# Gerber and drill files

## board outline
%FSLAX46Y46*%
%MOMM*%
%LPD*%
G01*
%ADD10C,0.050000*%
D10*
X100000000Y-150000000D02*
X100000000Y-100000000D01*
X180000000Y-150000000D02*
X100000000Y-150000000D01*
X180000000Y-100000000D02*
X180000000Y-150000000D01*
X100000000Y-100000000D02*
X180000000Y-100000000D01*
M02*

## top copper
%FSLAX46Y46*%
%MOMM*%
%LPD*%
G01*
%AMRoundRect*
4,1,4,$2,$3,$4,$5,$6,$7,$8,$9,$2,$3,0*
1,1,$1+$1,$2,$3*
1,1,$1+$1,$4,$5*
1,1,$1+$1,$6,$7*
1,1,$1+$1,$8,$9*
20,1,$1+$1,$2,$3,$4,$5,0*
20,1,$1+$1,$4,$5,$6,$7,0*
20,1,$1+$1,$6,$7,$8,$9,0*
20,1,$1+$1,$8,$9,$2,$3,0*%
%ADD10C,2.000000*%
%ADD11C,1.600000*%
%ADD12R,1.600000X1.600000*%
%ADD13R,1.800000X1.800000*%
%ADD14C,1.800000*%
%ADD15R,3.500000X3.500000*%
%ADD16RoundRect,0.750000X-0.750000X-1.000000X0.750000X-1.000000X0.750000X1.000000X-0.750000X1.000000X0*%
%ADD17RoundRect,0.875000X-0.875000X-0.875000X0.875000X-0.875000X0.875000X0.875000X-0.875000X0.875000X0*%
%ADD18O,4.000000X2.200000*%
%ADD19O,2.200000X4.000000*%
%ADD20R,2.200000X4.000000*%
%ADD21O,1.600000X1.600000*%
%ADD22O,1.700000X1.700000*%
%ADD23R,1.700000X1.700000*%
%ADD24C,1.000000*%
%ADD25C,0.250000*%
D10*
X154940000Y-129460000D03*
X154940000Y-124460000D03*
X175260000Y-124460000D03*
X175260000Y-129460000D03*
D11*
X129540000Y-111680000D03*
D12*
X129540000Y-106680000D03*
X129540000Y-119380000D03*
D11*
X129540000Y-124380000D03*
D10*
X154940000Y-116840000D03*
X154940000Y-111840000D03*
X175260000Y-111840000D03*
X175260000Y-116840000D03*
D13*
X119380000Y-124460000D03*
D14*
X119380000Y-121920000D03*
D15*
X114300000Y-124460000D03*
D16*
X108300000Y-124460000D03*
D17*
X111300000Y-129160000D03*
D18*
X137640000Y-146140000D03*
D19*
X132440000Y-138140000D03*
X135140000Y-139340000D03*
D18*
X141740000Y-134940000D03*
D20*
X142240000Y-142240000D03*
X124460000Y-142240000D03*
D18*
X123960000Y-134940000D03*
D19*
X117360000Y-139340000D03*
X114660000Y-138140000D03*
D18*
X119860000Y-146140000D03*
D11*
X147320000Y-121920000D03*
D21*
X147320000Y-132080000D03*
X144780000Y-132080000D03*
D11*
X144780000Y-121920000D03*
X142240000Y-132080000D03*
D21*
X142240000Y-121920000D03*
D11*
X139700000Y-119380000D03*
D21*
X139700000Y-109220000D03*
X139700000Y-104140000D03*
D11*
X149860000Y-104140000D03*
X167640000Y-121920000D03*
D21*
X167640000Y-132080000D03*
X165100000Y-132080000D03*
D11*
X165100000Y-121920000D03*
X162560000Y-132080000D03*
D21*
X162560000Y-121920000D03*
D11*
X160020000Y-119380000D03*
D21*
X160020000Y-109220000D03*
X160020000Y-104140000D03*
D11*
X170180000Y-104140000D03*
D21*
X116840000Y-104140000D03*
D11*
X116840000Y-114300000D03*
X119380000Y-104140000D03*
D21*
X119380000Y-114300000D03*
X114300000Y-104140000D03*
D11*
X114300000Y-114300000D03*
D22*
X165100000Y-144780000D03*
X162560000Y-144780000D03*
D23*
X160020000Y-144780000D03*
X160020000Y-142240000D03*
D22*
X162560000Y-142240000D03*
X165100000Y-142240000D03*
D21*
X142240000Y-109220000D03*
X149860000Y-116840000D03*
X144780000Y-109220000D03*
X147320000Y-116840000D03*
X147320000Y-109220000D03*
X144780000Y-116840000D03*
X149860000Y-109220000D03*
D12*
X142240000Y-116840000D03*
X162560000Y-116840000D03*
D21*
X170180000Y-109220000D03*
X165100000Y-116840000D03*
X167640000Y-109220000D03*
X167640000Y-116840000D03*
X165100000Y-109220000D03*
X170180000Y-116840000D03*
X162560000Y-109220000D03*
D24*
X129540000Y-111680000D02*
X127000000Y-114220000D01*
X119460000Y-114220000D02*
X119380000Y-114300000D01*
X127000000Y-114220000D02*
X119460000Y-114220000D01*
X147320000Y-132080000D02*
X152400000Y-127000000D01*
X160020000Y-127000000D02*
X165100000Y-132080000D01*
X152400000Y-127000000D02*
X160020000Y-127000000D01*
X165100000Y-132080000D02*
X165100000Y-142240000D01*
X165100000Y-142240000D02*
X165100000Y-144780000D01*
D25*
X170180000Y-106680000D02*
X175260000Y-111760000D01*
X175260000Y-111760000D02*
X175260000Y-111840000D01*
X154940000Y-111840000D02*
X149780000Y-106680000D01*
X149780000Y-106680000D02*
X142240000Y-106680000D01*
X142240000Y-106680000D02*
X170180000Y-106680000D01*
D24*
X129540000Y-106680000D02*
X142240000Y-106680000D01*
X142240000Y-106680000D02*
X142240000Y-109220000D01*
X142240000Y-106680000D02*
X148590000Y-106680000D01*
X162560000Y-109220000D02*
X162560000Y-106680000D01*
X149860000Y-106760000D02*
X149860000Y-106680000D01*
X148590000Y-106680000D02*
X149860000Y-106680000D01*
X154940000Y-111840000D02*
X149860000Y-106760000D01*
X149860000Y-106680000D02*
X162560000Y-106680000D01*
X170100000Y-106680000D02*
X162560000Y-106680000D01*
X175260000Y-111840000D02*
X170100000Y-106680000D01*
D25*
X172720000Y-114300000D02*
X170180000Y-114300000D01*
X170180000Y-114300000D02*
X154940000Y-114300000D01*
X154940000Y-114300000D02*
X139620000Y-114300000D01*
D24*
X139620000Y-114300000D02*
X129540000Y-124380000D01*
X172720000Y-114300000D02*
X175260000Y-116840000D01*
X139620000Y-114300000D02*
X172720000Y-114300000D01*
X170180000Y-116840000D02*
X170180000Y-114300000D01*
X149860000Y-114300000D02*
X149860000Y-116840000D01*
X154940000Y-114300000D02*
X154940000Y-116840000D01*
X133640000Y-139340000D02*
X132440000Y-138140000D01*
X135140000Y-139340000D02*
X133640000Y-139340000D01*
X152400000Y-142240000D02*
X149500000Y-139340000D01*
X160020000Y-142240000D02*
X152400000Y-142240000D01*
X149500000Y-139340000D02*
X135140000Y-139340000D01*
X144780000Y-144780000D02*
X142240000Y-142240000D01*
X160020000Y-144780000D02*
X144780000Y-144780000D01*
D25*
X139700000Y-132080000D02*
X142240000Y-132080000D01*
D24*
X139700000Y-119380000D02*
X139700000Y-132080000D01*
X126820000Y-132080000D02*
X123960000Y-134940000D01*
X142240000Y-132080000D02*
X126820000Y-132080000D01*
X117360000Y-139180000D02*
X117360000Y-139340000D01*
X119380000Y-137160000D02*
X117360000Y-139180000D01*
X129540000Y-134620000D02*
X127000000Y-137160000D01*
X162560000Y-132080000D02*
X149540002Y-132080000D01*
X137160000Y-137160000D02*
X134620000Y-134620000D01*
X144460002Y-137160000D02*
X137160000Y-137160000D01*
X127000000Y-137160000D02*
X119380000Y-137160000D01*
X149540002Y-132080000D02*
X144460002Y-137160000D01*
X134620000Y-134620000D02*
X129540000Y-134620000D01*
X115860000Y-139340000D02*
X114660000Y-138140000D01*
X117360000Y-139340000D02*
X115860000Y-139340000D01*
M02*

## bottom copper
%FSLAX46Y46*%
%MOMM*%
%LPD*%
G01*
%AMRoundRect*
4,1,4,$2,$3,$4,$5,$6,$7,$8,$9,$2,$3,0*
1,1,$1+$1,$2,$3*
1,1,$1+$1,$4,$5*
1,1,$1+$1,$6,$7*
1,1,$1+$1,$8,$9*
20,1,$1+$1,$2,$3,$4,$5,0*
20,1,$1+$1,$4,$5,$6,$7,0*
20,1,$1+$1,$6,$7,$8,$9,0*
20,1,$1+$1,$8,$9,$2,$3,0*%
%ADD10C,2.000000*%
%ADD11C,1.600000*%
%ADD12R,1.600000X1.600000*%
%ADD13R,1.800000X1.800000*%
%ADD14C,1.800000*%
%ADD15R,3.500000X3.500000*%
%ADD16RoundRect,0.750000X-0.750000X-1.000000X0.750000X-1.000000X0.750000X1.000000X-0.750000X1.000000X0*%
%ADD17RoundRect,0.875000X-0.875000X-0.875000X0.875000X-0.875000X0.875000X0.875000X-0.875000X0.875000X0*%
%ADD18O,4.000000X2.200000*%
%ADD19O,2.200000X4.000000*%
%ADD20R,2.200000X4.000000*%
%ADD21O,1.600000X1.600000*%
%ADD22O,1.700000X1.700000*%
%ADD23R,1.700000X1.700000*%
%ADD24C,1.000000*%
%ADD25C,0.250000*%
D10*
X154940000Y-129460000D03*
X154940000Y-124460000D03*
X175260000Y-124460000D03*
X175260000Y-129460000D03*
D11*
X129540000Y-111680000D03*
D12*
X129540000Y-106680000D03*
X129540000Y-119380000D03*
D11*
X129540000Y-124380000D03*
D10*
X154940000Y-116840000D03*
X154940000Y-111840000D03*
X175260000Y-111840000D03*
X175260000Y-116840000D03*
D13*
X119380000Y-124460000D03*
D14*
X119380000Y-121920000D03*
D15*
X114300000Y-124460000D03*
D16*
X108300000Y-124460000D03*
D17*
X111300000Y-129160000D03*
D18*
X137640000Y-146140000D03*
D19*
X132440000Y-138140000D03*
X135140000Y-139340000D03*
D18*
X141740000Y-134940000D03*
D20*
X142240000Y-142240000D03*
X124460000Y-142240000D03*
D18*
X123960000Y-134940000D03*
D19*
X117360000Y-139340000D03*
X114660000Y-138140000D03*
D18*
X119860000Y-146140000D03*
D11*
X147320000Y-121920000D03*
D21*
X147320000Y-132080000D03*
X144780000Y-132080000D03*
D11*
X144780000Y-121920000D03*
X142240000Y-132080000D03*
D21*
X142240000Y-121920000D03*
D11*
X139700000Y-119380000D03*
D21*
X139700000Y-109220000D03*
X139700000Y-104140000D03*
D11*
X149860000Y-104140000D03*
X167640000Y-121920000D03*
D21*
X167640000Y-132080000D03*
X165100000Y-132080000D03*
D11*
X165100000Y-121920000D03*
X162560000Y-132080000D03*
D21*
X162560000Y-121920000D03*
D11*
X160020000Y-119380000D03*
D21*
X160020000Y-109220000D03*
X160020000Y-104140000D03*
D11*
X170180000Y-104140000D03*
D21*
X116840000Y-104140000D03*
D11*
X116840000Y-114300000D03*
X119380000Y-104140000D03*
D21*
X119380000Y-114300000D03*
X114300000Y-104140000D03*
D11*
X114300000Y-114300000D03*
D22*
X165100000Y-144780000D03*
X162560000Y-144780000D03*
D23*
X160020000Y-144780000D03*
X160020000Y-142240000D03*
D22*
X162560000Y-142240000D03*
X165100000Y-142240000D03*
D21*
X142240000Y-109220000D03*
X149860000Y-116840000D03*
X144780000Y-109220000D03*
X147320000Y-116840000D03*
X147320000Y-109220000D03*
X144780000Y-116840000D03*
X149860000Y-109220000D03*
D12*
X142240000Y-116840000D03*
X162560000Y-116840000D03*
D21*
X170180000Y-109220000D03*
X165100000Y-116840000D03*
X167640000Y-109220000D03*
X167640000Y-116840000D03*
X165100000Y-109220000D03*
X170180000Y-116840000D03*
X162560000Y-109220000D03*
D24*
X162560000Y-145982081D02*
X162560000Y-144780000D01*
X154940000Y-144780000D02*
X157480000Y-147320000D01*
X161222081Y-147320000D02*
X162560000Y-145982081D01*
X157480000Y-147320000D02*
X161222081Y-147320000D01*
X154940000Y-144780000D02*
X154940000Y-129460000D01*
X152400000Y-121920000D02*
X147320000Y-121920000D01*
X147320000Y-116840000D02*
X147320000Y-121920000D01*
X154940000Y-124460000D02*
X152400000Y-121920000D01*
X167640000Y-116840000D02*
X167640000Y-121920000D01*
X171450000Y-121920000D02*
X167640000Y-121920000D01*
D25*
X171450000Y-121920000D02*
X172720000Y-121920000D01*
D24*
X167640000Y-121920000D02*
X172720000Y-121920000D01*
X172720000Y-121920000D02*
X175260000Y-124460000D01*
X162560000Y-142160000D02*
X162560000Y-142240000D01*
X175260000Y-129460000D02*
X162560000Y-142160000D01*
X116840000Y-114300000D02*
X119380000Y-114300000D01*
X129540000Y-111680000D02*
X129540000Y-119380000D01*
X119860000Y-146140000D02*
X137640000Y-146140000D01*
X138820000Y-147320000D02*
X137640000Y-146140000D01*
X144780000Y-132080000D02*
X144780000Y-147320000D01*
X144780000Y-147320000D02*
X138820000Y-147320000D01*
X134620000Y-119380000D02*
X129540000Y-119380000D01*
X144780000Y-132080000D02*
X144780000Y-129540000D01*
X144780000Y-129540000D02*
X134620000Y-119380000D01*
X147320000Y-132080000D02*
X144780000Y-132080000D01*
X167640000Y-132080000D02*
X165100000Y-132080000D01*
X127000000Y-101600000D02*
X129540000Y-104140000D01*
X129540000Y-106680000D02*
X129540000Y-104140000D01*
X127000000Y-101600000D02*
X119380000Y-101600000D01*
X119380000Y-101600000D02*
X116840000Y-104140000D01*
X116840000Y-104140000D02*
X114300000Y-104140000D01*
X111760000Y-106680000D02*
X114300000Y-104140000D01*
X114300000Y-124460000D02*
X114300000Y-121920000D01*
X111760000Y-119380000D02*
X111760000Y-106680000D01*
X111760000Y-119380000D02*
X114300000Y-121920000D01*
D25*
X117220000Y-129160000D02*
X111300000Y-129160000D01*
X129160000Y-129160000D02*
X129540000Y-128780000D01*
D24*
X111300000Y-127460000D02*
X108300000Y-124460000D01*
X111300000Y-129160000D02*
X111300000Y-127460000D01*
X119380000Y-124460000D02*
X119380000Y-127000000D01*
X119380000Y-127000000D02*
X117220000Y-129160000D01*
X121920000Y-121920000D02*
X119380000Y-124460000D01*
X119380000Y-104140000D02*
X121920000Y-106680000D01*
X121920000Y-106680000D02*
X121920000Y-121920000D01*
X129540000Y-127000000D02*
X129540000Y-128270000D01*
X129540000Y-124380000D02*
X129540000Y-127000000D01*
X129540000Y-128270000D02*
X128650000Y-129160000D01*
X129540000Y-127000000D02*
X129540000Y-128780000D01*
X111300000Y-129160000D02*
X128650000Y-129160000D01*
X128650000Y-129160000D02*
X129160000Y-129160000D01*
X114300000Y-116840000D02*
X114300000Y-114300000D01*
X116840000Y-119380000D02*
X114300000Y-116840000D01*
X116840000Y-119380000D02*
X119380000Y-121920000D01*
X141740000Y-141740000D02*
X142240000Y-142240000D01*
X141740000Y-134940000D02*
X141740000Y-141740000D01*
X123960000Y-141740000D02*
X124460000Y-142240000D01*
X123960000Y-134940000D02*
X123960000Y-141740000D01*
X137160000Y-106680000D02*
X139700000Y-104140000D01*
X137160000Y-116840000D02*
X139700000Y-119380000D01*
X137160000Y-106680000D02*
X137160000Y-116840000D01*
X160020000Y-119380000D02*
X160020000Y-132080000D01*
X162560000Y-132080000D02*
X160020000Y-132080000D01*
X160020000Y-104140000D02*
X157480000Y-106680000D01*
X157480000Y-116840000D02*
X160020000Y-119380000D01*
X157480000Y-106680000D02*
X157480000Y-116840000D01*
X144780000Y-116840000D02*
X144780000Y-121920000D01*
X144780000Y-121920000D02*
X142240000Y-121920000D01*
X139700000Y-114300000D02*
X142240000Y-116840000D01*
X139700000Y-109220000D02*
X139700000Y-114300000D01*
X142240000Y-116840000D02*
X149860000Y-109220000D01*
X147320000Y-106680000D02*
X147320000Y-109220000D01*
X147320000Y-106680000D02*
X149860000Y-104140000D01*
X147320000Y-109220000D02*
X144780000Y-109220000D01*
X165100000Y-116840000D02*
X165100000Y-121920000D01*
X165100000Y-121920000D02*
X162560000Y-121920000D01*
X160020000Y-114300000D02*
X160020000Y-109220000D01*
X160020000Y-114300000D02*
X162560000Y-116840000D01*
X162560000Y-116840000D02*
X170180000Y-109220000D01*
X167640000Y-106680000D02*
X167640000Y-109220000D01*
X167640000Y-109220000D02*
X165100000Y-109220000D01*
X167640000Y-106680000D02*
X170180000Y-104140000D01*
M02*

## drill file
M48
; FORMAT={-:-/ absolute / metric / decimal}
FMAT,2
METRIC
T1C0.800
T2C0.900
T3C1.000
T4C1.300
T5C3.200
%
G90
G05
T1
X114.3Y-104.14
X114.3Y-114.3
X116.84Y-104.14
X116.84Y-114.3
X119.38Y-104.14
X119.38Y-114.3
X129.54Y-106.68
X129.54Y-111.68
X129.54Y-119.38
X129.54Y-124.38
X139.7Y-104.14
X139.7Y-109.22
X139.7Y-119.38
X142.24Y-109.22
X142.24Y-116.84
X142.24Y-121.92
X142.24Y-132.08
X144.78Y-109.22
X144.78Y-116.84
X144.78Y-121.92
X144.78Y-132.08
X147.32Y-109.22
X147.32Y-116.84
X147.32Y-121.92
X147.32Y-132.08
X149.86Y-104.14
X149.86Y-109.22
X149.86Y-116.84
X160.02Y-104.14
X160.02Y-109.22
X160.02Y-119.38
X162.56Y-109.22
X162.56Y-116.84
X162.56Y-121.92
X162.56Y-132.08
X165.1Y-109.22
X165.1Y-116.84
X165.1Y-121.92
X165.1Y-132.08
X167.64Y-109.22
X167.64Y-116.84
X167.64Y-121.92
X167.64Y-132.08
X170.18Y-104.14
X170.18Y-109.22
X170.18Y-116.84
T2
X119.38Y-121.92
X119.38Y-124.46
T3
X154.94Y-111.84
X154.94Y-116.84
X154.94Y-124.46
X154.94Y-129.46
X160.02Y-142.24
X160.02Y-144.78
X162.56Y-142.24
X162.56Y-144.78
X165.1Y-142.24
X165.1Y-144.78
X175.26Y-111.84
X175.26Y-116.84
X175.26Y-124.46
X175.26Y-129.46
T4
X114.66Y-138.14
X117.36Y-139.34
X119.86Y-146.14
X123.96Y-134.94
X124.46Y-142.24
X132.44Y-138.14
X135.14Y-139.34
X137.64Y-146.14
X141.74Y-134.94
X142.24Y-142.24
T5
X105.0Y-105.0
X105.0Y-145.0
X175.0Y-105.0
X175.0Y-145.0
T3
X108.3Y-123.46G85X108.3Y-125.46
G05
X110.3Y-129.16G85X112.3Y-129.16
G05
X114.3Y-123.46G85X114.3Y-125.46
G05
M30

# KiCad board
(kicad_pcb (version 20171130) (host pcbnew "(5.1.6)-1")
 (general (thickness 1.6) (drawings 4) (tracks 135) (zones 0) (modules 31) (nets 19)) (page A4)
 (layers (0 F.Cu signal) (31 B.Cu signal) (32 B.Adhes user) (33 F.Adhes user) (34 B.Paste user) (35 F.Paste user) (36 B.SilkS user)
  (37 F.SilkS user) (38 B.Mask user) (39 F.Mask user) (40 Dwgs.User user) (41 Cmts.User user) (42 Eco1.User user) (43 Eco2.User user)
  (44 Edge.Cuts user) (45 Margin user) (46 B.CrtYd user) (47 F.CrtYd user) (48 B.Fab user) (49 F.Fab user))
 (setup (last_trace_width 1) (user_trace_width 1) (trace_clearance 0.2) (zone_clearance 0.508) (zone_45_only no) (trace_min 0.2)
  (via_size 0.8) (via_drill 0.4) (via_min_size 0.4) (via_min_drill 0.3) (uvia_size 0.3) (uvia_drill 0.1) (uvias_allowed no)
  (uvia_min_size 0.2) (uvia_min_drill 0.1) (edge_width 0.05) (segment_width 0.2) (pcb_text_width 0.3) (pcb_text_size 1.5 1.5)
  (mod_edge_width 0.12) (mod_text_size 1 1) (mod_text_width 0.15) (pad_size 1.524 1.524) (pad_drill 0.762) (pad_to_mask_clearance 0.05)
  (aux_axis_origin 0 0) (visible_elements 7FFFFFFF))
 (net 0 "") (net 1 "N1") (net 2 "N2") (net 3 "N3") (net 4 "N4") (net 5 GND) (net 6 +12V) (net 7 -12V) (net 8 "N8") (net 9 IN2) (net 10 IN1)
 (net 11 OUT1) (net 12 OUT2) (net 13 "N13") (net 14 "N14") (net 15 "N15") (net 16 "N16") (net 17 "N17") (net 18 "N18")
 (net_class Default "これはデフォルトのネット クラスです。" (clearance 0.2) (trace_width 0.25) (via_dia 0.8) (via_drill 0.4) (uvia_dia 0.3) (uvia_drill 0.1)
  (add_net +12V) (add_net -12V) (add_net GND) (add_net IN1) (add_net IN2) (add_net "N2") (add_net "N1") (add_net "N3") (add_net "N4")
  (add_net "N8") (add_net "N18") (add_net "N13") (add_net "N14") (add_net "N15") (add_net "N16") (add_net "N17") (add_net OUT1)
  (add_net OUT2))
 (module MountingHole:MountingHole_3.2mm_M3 (layer F.Cu) (at 175 105)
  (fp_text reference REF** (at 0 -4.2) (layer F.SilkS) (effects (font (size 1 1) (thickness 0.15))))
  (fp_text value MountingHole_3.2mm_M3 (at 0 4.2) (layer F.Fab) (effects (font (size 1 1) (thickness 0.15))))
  (pad 1 np_thru_hole circle (at 0 0) (size 3.2 3.2) (drill 3.2) (layers *.Cu *.Mask)))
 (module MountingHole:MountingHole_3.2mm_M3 (layer F.Cu) (at 175 145)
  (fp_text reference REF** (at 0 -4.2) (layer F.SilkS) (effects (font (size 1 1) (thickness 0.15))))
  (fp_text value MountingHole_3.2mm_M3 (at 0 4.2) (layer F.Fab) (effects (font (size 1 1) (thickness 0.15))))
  (pad 1 np_thru_hole circle (at 0 0) (size 3.2 3.2) (drill 3.2) (layers *.Cu *.Mask)))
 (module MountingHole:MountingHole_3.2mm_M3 (layer F.Cu) (at 105 145)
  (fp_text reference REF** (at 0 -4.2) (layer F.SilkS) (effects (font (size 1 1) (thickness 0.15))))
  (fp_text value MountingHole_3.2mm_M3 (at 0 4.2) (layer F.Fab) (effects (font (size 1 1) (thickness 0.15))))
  (pad 1 np_thru_hole circle (at 0 0) (size 3.2 3.2) (drill 3.2) (layers *.Cu *.Mask)))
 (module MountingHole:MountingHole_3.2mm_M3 (layer F.Cu) (at 105 105)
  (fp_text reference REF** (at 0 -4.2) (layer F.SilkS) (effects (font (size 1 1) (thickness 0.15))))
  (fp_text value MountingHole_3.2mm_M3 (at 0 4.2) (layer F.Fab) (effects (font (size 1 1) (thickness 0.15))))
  (pad 1 np_thru_hole circle (at 0 0) (size 3.2 3.2) (drill 3.2) (layers *.Cu *.Mask)))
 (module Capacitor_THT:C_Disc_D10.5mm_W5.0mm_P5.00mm (layer F.Cu) (at 154.94 124.46 270)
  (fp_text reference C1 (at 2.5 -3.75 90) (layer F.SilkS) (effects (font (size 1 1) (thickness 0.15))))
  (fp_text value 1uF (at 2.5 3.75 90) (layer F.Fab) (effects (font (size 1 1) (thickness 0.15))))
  (pad 2 thru_hole circle (at 5 0 270) (size 2 2) (drill 1) (layers *.Cu *.Mask) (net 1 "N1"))
  (pad 1 thru_hole circle (at 0 0 270) (size 2 2) (drill 1) (layers *.Cu *.Mask) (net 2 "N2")))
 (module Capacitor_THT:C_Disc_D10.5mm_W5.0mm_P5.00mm (layer F.Cu) (at 175.26 124.46 270)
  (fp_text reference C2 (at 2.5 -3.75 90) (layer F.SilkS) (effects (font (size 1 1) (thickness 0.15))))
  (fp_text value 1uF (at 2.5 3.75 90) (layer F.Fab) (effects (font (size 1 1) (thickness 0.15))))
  (pad 1 thru_hole circle (at 0 0 270) (size 2 2) (drill 1) (layers *.Cu *.Mask) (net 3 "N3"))
  (pad 2 thru_hole circle (at 5 0 270) (size 2 2) (drill 1) (layers *.Cu *.Mask) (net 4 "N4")))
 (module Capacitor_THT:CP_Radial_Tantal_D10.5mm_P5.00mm (layer F.Cu) (at 129.54 106.68 270)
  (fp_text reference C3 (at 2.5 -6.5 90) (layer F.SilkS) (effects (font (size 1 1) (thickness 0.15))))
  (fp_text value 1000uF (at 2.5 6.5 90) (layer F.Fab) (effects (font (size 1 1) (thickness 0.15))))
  (pad 2 thru_hole circle (at 5 0 270) (size 1.6 1.6) (drill 0.8) (layers *.Cu *.Mask) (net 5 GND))
  (pad 1 thru_hole rect (at 0 0 270) (size 1.6 1.6) (drill 0.8) (layers *.Cu *.Mask) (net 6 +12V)))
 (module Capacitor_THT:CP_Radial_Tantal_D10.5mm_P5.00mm (layer F.Cu) (at 129.54 119.38 270)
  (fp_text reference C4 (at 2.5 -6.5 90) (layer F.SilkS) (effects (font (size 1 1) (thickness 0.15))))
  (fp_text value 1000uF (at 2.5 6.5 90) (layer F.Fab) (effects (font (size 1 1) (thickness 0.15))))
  (pad 1 thru_hole rect (at 0 0 270) (size 1.6 1.6) (drill 0.8) (layers *.Cu *.Mask) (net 5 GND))
  (pad 2 thru_hole circle (at 5 0 270) (size 1.6 1.6) (drill 0.8) (layers *.Cu *.Mask) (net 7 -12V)))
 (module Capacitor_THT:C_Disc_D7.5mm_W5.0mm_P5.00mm (layer F.Cu) (at 154.94 116.84 90)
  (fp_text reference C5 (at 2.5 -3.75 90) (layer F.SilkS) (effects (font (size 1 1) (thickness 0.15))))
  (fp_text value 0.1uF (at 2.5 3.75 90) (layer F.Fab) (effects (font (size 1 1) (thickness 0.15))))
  (pad 1 thru_hole circle (at 0 0 90) (size 2 2) (drill 1) (layers *.Cu *.Mask) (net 7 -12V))
  (pad 2 thru_hole circle (at 5 0 90) (size 2 2) (drill 1) (layers *.Cu *.Mask) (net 6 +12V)))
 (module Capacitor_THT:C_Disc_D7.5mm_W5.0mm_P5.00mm (layer F.Cu) (at 175.26 116.84 90)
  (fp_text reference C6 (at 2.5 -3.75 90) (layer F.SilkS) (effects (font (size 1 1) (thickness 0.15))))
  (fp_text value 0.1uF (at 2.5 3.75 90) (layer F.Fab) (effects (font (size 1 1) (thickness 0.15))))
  (pad 2 thru_hole circle (at 5 0 90) (size 2 2) (drill 1) (layers *.Cu *.Mask) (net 6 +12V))
  (pad 1 thru_hole circle (at 0 0 90) (size 2 2) (drill 1) (layers *.Cu *.Mask) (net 7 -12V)))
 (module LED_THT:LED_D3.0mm (layer F.Cu) (at 119.38 124.46 90)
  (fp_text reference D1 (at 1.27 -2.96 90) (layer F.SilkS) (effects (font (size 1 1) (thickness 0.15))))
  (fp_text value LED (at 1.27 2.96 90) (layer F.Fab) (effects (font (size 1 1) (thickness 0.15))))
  (pad 1 thru_hole rect (at 0 0 90) (size 1.8 1.8) (drill 0.9) (layers *.Cu *.Mask) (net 7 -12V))
  (pad 2 thru_hole circle (at 2.54 0 90) (size 1.8 1.8) (drill 0.9) (layers *.Cu *.Mask) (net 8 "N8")))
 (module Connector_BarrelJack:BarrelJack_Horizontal (layer F.Cu) (at 114.3 124.46)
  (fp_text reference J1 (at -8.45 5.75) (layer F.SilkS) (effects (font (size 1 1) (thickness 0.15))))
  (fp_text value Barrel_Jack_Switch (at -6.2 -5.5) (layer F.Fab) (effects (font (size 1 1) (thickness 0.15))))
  (pad 1 thru_hole rect (at 0 0) (size 3.5 3.5) (drill oval 1 3) (layers *.Cu *.Mask) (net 6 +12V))
  (pad 2 thru_hole roundrect (at -6 0) (size 3 3.5) (drill oval 1 3) (layers *.Cu *.Mask) (roundrect_rratio 0.25) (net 7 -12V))
  (pad 3 thru_hole roundrect (at -3 4.7) (size 3.5 3.5) (drill oval 3 1) (layers *.Cu *.Mask) (roundrect_rratio 0.25) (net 7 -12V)))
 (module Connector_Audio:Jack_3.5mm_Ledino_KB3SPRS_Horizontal (layer F.Cu) (at 142.24 142.24 90)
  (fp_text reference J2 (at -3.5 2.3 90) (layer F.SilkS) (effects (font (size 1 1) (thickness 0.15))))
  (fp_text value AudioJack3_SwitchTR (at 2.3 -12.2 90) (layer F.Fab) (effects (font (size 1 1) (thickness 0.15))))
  (pad S thru_hole oval (at -3.9 -4.6 90) (size 2.2 4) (drill 1.3) (layers *.Cu *.Mask) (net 5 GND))
  (pad R thru_hole oval (at 4.1 -9.8 90) (size 4 2.2) (drill 1.3) (layers *.Cu *.Mask) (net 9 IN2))
  (pad RN thru_hole oval (at 2.9 -7.1 90) (size 4 2.2) (drill 1.3) (layers *.Cu *.Mask) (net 9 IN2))
  (pad TN thru_hole oval (at 7.3 -0.5 180) (size 4 2.2) (drill 1.3) (layers *.Cu *.Mask) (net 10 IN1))
  (pad T thru_hole rect (at 0 0 90) (size 4 2.2) (drill 1.3) (layers *.Cu *.Mask) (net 10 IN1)))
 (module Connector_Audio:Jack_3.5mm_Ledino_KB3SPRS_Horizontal (layer F.Cu) (at 124.46 142.24 90)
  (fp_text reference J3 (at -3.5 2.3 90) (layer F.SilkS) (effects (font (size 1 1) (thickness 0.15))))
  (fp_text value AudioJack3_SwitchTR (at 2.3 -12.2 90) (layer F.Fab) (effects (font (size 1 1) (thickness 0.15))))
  (pad T thru_hole rect (at 0 0 90) (size 4 2.2) (drill 1.3) (layers *.Cu *.Mask) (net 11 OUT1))
  (pad TN thru_hole oval (at 7.3 -0.5 180) (size 4 2.2) (drill 1.3) (layers *.Cu *.Mask) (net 11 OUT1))
  (pad RN thru_hole oval (at 2.9 -7.1 90) (size 4 2.2) (drill 1.3) (layers *.Cu *.Mask) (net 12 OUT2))
  (pad R thru_hole oval (at 4.1 -9.8 90) (size 4 2.2) (drill 1.3) (layers *.Cu *.Mask) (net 12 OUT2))
  (pad S thru_hole oval (at -3.9 -4.6 90) (size 2.2 4) (drill 1.3) (layers *.Cu *.Mask) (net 5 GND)))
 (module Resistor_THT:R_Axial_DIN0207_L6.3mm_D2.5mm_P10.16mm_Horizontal (layer F.Cu) (at 147.32 121.92 270)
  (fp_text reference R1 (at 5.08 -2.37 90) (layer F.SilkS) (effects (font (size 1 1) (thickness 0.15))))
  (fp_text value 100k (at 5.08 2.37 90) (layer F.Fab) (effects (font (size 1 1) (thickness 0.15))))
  (pad 1 thru_hole circle (at 0 0 270) (size 1.6 1.6) (drill 0.8) (layers *.Cu *.Mask) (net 2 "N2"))
  (pad 2 thru_hole oval (at 10.16 0 270) (size 1.6 1.6) (drill 0.8) (layers *.Cu *.Mask) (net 5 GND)))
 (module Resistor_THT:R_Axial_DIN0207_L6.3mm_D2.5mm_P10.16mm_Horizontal (layer F.Cu) (at 144.78 121.92 270)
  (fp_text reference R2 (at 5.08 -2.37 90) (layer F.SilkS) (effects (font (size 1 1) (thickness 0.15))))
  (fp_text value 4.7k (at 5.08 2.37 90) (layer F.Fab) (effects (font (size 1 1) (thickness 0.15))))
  (pad 2 thru_hole oval (at 10.16 0 270) (size 1.6 1.6) (drill 0.8) (layers *.Cu *.Mask) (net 5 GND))
  (pad 1 thru_hole circle (at 0 0 270) (size 1.6 1.6) (drill 0.8) (layers *.Cu *.Mask) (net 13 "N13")))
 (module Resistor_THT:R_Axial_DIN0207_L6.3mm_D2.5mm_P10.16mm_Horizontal (layer F.Cu) (at 142.24 132.08 90)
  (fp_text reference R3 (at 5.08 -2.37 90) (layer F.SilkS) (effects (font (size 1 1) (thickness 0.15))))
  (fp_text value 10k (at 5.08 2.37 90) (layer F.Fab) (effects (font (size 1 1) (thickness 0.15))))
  (pad 1 thru_hole circle (at 0 0 90) (size 1.6 1.6) (drill 0.8) (layers *.Cu *.Mask) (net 11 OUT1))
  (pad 2 thru_hole oval (at 10.16 0 90) (size 1.6 1.6) (drill 0.8) (layers *.Cu *.Mask) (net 13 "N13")))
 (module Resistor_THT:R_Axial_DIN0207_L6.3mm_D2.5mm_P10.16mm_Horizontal (layer F.Cu) (at 139.7 119.38 90)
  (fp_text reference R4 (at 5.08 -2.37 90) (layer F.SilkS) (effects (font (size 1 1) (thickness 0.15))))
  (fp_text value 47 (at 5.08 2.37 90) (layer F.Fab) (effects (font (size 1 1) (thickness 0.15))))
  (pad 1 thru_hole circle (at 0 0 90) (size 1.6 1.6) (drill 0.8) (layers *.Cu *.Mask) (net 11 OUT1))
  (pad 2 thru_hole oval (at 10.16 0 90) (size 1.6 1.6) (drill 0.8) (layers *.Cu *.Mask) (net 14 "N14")))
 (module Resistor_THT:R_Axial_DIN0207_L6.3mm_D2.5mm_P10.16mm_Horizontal (layer F.Cu) (at 149.86 104.14 180)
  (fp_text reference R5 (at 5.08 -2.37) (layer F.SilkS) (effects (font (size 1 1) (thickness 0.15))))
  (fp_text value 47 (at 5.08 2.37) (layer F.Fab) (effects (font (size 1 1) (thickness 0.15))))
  (pad 2 thru_hole oval (at 10.16 0 180) (size 1.6 1.6) (drill 0.8) (layers *.Cu *.Mask) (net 11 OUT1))
  (pad 1 thru_hole circle (at 0 0 180) (size 1.6 1.6) (drill 0.8) (layers *.Cu *.Mask) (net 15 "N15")))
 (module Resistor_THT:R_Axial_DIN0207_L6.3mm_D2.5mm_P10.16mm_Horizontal (layer F.Cu) (at 167.64 121.92 270)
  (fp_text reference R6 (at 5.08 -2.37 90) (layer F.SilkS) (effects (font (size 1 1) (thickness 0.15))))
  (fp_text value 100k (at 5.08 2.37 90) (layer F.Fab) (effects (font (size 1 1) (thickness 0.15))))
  (pad 1 thru_hole circle (at 0 0 270) (size 1.6 1.6) (drill 0.8) (layers *.Cu *.Mask) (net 3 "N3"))
  (pad 2 thru_hole oval (at 10.16 0 270) (size 1.6 1.6) (drill 0.8) (layers *.Cu *.Mask) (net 5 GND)))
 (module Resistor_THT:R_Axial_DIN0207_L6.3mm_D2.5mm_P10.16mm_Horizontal (layer F.Cu) (at 165.1 121.92 270)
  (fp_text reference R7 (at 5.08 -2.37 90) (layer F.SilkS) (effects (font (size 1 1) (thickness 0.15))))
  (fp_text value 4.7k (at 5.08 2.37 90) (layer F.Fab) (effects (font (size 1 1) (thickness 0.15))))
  (pad 2 thru_hole oval (at 10.16 0 270) (size 1.6 1.6) (drill 0.8) (layers *.Cu *.Mask) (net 5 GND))
  (pad 1 thru_hole circle (at 0 0 270) (size 1.6 1.6) (drill 0.8) (layers *.Cu *.Mask) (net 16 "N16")))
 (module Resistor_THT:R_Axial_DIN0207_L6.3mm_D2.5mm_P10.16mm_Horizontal (layer F.Cu) (at 162.56 132.08 90)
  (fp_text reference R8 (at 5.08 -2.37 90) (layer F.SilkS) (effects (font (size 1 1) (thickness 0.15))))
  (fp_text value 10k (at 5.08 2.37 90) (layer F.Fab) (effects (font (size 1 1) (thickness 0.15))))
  (pad 1 thru_hole circle (at 0 0 90) (size 1.6 1.6) (drill 0.8) (layers *.Cu *.Mask) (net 12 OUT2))
  (pad 2 thru_hole oval (at 10.16 0 90) (size 1.6 1.6) (drill 0.8) (layers *.Cu *.Mask) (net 16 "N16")))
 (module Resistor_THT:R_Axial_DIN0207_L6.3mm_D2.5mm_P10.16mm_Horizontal (layer F.Cu) (at 160.02 119.38 90)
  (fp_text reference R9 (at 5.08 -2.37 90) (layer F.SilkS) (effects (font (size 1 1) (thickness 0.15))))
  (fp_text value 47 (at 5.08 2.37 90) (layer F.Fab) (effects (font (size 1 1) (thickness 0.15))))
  (pad 1 thru_hole circle (at 0 0 90) (size 1.6 1.6) (drill 0.8) (layers *.Cu *.Mask) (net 12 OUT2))
  (pad 2 thru_hole oval (at 10.16 0 90) (size 1.6 1.6) (drill 0.8) (layers *.Cu *.Mask) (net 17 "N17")))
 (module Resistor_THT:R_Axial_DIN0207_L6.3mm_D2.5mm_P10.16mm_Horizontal (layer F.Cu) (at 170.18 104.14 180)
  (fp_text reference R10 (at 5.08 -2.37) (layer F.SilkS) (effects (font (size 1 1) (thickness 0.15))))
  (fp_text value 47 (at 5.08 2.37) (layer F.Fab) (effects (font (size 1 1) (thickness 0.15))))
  (pad 2 thru_hole oval (at 10.16 0 180) (size 1.6 1.6) (drill 0.8) (layers *.Cu *.Mask) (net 12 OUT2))
  (pad 1 thru_hole circle (at 0 0 180) (size 1.6 1.6) (drill 0.8) (layers *.Cu *.Mask) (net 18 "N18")))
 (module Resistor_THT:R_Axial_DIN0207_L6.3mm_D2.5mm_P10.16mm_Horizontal (layer F.Cu) (at 116.84 114.3 90)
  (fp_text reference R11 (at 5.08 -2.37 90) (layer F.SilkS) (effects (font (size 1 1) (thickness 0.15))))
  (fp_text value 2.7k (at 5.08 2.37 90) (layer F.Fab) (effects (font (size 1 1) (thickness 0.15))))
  (pad 2 thru_hole oval (at 10.16 0 90) (size 1.6 1.6) (drill 0.8) (layers *.Cu *.Mask) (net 6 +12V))
  (pad 1 thru_hole circle (at 0 0 90) (size 1.6 1.6) (drill 0.8) (layers *.Cu *.Mask) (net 5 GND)))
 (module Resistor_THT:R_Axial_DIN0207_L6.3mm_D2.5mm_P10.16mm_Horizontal (layer F.Cu) (at 119.38 104.14 270)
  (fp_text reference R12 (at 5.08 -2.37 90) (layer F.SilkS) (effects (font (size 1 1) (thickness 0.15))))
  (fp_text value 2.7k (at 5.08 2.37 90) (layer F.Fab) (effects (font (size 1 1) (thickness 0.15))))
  (pad 1 thru_hole circle (at 0 0 270) (size 1.6 1.6) (drill 0.8) (layers *.Cu *.Mask) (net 7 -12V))
  (pad 2 thru_hole oval (at 10.16 0 270) (size 1.6 1.6) (drill 0.8) (layers *.Cu *.Mask) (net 5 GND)))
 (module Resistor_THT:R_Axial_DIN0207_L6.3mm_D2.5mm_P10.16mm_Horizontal (layer F.Cu) (at 114.3 114.3 90)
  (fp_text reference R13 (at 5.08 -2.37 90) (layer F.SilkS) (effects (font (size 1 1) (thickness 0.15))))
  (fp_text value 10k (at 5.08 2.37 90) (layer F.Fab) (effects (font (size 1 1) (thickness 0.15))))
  (pad 2 thru_hole oval (at 10.16 0 90) (size 1.6 1.6) (drill 0.8) (layers *.Cu *.Mask) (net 6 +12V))
  (pad 1 thru_hole circle (at 0 0 90) (size 1.6 1.6) (drill 0.8) (layers *.Cu *.Mask) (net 8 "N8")))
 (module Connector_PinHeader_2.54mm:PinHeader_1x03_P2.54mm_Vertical (layer F.Cu) (at 160.02 144.78 90)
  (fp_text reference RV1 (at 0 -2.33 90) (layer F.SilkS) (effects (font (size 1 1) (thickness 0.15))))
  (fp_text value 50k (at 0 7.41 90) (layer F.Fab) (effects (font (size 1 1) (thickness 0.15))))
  (pad 3 thru_hole oval (at 0 5.08 90) (size 1.7 1.7) (drill 1) (layers *.Cu *.Mask) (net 5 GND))
  (pad 2 thru_hole oval (at 0 2.54 90) (size 1.7 1.7) (drill 1) (layers *.Cu *.Mask) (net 1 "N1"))
  (pad 1 thru_hole rect (at 0 0 90) (size 1.7 1.7) (drill 1) (layers *.Cu *.Mask) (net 10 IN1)))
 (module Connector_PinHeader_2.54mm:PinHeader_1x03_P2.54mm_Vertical (layer F.Cu) (at 160.02 142.24 90)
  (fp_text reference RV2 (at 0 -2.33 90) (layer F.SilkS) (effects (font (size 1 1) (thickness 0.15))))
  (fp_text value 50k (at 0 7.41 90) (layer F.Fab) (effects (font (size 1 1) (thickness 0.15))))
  (pad 1 thru_hole rect (at 0 0 90) (size 1.7 1.7) (drill 1) (layers *.Cu *.Mask) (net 9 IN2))
  (pad 2 thru_hole oval (at 0 2.54 90) (size 1.7 1.7) (drill 1) (layers *.Cu *.Mask) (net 4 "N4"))
  (pad 3 thru_hole oval (at 0 5.08 90) (size 1.7 1.7) (drill 1) (layers *.Cu *.Mask) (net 5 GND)))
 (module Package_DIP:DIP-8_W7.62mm (layer F.Cu) (at 142.24 116.84 90)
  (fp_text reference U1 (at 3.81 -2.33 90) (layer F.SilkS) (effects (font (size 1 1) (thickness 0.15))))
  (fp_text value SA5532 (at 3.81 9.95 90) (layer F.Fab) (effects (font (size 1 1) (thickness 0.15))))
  (pad 8 thru_hole oval (at 7.62 0 90) (size 1.6 1.6) (drill 0.8) (layers *.Cu *.Mask) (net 6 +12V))
  (pad 4 thru_hole oval (at 0 7.62 90) (size 1.6 1.6) (drill 0.8) (layers *.Cu *.Mask) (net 7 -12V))
  (pad 7 thru_hole oval (at 7.62 2.54 90) (size 1.6 1.6) (drill 0.8) (layers *.Cu *.Mask) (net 15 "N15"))
  (pad 3 thru_hole oval (at 0 5.08 90) (size 1.6 1.6) (drill 0.8) (layers *.Cu *.Mask) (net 2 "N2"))
  (pad 6 thru_hole oval (at 7.62 5.08 90) (size 1.6 1.6) (drill 0.8) (layers *.Cu *.Mask) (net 15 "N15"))
  (pad 2 thru_hole oval (at 0 2.54 90) (size 1.6 1.6) (drill 0.8) (layers *.Cu *.Mask) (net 13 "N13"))
  (pad 5 thru_hole oval (at 7.62 7.62 90) (size 1.6 1.6) (drill 0.8) (layers *.Cu *.Mask) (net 14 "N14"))
  (pad 1 thru_hole rect (at 0 0 90) (size 1.6 1.6) (drill 0.8) (layers *.Cu *.Mask) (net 14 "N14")))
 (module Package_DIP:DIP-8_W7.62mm (layer F.Cu) (at 162.56 116.84 90)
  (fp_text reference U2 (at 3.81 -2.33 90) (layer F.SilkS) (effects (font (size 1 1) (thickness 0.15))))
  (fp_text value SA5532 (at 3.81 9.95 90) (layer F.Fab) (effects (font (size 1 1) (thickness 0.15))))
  (pad 1 thru_hole rect (at 0 0 90) (size 1.6 1.6) (drill 0.8) (layers *.Cu *.Mask) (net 17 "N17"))
  (pad 5 thru_hole oval (at 7.62 7.62 90) (size 1.6 1.6) (drill 0.8) (layers *.Cu *.Mask) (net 17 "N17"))
  (pad 2 thru_hole oval (at 0 2.54 90) (size 1.6 1.6) (drill 0.8) (layers *.Cu *.Mask) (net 16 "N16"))
  (pad 6 thru_hole oval (at 7.62 5.08 90) (size 1.6 1.6) (drill 0.8) (layers *.Cu *.Mask) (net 18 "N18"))
  (pad 3 thru_hole oval (at 0 5.08 90) (size 1.6 1.6) (drill 0.8) (layers *.Cu *.Mask) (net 3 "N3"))
  (pad 7 thru_hole oval (at 7.62 2.54 90) (size 1.6 1.6) (drill 0.8) (layers *.Cu *.Mask) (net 18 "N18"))
  (pad 4 thru_hole oval (at 0 7.62 90) (size 1.6 1.6) (drill 0.8) (layers *.Cu *.Mask) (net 7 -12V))
  (pad 8 thru_hole oval (at 7.62 0 90) (size 1.6 1.6) (drill 0.8) (layers *.Cu *.Mask) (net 6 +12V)))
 (gr_line (start 100 150) (end 100 100) (layer Edge.Cuts) (width 0.05))
 (gr_line (start 180 150) (end 100 150) (layer Edge.Cuts) (width 0.05))
 (gr_line (start 180 100) (end 180 150) (layer Edge.Cuts) (width 0.05))
 (gr_line (start 100 100) (end 180 100) (layer Edge.Cuts) (width 0.05))
 (segment (start 162.56 145.982081) (end 162.56 144.78) (width 1) (layer B.Cu) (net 1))
 (segment (start 154.94 144.78) (end 157.48 147.32) (width 1) (layer B.Cu) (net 1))
 (segment (start 161.222081 147.32) (end 162.56 145.982081) (width 1) (layer B.Cu) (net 1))
 (segment (start 157.48 147.32) (end 161.222081 147.32) (width 1) (layer B.Cu) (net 1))
 (segment (start 154.94 144.78) (end 154.94 129.46) (width 1) (layer B.Cu) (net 1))
 (segment (start 152.4 121.92) (end 147.32 121.92) (width 1) (layer B.Cu) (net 2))
 (segment (start 147.32 116.84) (end 147.32 121.92) (width 1) (layer B.Cu) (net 2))
 (segment (start 154.94 124.46) (end 152.4 121.92) (width 1) (layer B.Cu) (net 2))
 (segment (start 167.64 116.84) (end 167.64 121.92) (width 1) (layer B.Cu) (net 3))
 (segment (start 171.45 121.92) (end 167.64 121.92) (width 1) (layer B.Cu) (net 3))
 (segment (start 171.45 121.92) (end 172.72 121.92) (width 0.25) (layer B.Cu) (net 3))
 (segment (start 167.64 121.92) (end 172.72 121.92) (width 1) (layer B.Cu) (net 3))
 (segment (start 172.72 121.92) (end 175.26 124.46) (width 1) (layer B.Cu) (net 3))
 (segment (start 162.56 142.16) (end 162.56 142.24) (width 1) (layer B.Cu) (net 4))
 (segment (start 175.26 129.46) (end 162.56 142.16) (width 1) (layer B.Cu) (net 4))
 (segment (start 116.84 114.3) (end 119.38 114.3) (width 1) (layer B.Cu) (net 5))
 (segment (start 129.54 111.68) (end 127 114.22) (width 1) (layer F.Cu) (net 5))
 (segment (start 119.46 114.22) (end 119.38 114.3) (width 1) (layer F.Cu) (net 5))
 (segment (start 127 114.22) (end 119.46 114.22) (width 1) (layer F.Cu) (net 5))
 (segment (start 129.54 111.68) (end 129.54 119.38) (width 1) (layer B.Cu) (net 5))
 (segment (start 119.86 146.14) (end 137.64 146.14) (width 1) (layer B.Cu) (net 5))
 (segment (start 138.82 147.32) (end 137.64 146.14) (width 1) (layer B.Cu) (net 5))
 (segment (start 144.78 132.08) (end 144.78 147.32) (width 1) (layer B.Cu) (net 5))
 (segment (start 144.78 147.32) (end 138.82 147.32) (width 1) (layer B.Cu) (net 5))
 (segment (start 134.62 119.38) (end 129.54 119.38) (width 1) (layer B.Cu) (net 5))
 (segment (start 144.78 132.08) (end 144.78 129.54) (width 1) (layer B.Cu) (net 5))
 (segment (start 144.78 129.54) (end 134.62 119.38) (width 1) (layer B.Cu) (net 5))
 (segment (start 147.32 132.08) (end 144.78 132.08) (width 1) (layer B.Cu) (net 5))
 (segment (start 167.64 132.08) (end 165.1 132.08) (width 1) (layer B.Cu) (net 5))
 (segment (start 147.32 132.08) (end 152.4 127) (width 1) (layer F.Cu) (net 5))
 (segment (start 160.02 127) (end 165.1 132.08) (width 1) (layer F.Cu) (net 5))
 (segment (start 152.4 127) (end 160.02 127) (width 1) (layer F.Cu) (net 5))
 (segment (start 165.1 132.08) (end 165.1 142.24) (width 1) (layer F.Cu) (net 5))
 (segment (start 165.1 142.24) (end 165.1 144.78) (width 1) (layer F.Cu) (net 5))
 (segment (start 170.18 106.68) (end 175.26 111.76) (width 0.25) (layer F.Cu) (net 6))
 (segment (start 175.26 111.76) (end 175.26 111.84) (width 0.25) (layer F.Cu) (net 6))
 (segment (start 154.94 111.84) (end 149.78 106.68) (width 0.25) (layer F.Cu) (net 6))
 (segment (start 149.78 106.68) (end 142.24 106.68) (width 0.25) (layer F.Cu) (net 6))
 (segment (start 142.24 106.68) (end 170.18 106.68) (width 0.25) (layer F.Cu) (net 6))
 (segment (start 127 101.6) (end 129.54 104.14) (width 1) (layer B.Cu) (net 6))
 (segment (start 129.54 106.68) (end 129.54 104.14) (width 1) (layer B.Cu) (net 6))
 (segment (start 127 101.6) (end 119.38 101.6) (width 1) (layer B.Cu) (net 6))
 (segment (start 119.38 101.6) (end 116.84 104.14) (width 1) (layer B.Cu) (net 6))
 (segment (start 116.84 104.14) (end 114.3 104.14) (width 1) (layer B.Cu) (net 6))
 (segment (start 111.76 106.68) (end 114.3 104.14) (width 1) (layer B.Cu) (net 6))
 (segment (start 114.3 124.46) (end 114.3 121.92) (width 1) (layer B.Cu) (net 6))
 (segment (start 111.76 119.38) (end 111.76 106.68) (width 1) (layer B.Cu) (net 6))
 (segment (start 111.76 119.38) (end 114.3 121.92) (width 1) (layer B.Cu) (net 6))
 (segment (start 129.54 106.68) (end 142.24 106.68) (width 1) (layer F.Cu) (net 6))
 (segment (start 142.24 106.68) (end 142.24 109.22) (width 1) (layer F.Cu) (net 6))
 (segment (start 142.24 106.68) (end 148.59 106.68) (width 1) (layer F.Cu) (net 6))
 (segment (start 162.56 109.22) (end 162.56 106.68) (width 1) (layer F.Cu) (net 6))
 (segment (start 149.86 106.76) (end 149.86 106.68) (width 1) (layer F.Cu) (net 6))
 (segment (start 148.59 106.68) (end 149.86 106.68) (width 1) (layer F.Cu) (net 6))
 (segment (start 154.94 111.84) (end 149.86 106.76) (width 1) (layer F.Cu) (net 6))
 (segment (start 149.86 106.68) (end 162.56 106.68) (width 1) (layer F.Cu) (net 6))
 (segment (start 170.1 106.68) (end 162.56 106.68) (width 1) (layer F.Cu) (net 6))
 (segment (start 175.26 111.84) (end 170.1 106.68) (width 1) (layer F.Cu) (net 6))
 (segment (start 117.22 129.16) (end 111.3 129.16) (width 0.25) (layer B.Cu) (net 7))
 (segment (start 129.16 129.16) (end 129.54 128.78) (width 0.25) (layer B.Cu) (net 7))
 (segment (start 172.72 114.3) (end 170.18 114.3) (width 0.25) (layer F.Cu) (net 7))
 (segment (start 170.18 114.3) (end 154.94 114.3) (width 0.25) (layer F.Cu) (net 7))
 (segment (start 154.94 114.3) (end 139.62 114.3) (width 0.25) (layer F.Cu) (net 7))
 (segment (start 111.3 127.46) (end 108.3 124.46) (width 1) (layer B.Cu) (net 7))
 (segment (start 111.3 129.16) (end 111.3 127.46) (width 1) (layer B.Cu) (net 7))
 (segment (start 119.38 124.46) (end 119.38 127) (width 1) (layer B.Cu) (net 7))
 (segment (start 119.38 127) (end 117.22 129.16) (width 1) (layer B.Cu) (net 7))
 (segment (start 121.92 121.92) (end 119.38 124.46) (width 1) (layer B.Cu) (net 7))
 (segment (start 119.38 104.14) (end 121.92 106.68) (width 1) (layer B.Cu) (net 7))
 (segment (start 121.92 106.68) (end 121.92 121.92) (width 1) (layer B.Cu) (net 7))
 (segment (start 139.62 114.3) (end 129.54 124.38) (width 1) (layer F.Cu) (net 7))
 (segment (start 172.72 114.3) (end 175.26 116.84) (width 1) (layer F.Cu) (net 7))
 (segment (start 139.62 114.3) (end 172.72 114.3) (width 1) (layer F.Cu) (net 7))
 (segment (start 170.18 116.84) (end 170.18 114.3) (width 1) (layer F.Cu) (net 7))
 (segment (start 149.86 114.3) (end 149.86 116.84) (width 1) (layer F.Cu) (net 7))
 (segment (start 154.94 114.3) (end 154.94 116.84) (width 1) (layer F.Cu) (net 7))
 (segment (start 129.54 127) (end 129.54 128.27) (width 1) (layer B.Cu) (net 7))
 (segment (start 129.54 124.38) (end 129.54 127) (width 1) (layer B.Cu) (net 7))
 (segment (start 129.54 128.27) (end 128.65 129.16) (width 1) (layer B.Cu) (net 7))
 (segment (start 129.54 127) (end 129.54 128.78) (width 1) (layer B.Cu) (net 7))
 (segment (start 111.3 129.16) (end 128.65 129.16) (width 1) (layer B.Cu) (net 7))
 (segment (start 128.65 129.16) (end 129.16 129.16) (width 1) (layer B.Cu) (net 7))
 (segment (start 114.3 116.84) (end 114.3 114.3) (width 1) (layer B.Cu) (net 8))
 (segment (start 116.84 119.38) (end 114.3 116.84) (width 1) (layer B.Cu) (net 8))
 (segment (start 116.84 119.38) (end 119.38 121.92) (width 1) (layer B.Cu) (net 8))
 (segment (start 133.64 139.34) (end 132.44 138.14) (width 1) (layer F.Cu) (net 9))
 (segment (start 135.14 139.34) (end 133.64 139.34) (width 1) (layer F.Cu) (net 9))
 (segment (start 152.4 142.24) (end 149.5 139.34) (width 1) (layer F.Cu) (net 9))
 (segment (start 160.02 142.24) (end 152.4 142.24) (width 1) (layer F.Cu) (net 9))
 (segment (start 149.5 139.34) (end 135.14 139.34) (width 1) (layer F.Cu) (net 9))
 (segment (start 141.74 141.74) (end 142.24 142.24) (width 1) (layer B.Cu) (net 10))
 (segment (start 141.74 134.94) (end 141.74 141.74) (width 1) (layer B.Cu) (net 10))
 (segment (start 144.78 144.78) (end 142.24 142.24) (width 1) (layer F.Cu) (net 10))
 (segment (start 160.02 144.78) (end 144.78 144.78) (width 1) (layer F.Cu) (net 10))
 (segment (start 139.7 132.08) (end 142.24 132.08) (width 0.25) (layer F.Cu) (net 11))
 (segment (start 123.96 141.74) (end 124.46 142.24) (width 1) (layer B.Cu) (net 11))
 (segment (start 123.96 134.94) (end 123.96 141.74) (width 1) (layer B.Cu) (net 11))
 (segment (start 137.16 106.68) (end 139.7 104.14) (width 1) (layer B.Cu) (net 11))
 (segment (start 137.16 116.84) (end 139.7 119.38) (width 1) (layer B.Cu) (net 11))
 (segment (start 137.16 106.68) (end 137.16 116.84) (width 1) (layer B.Cu) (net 11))
 (segment (start 139.7 119.38) (end 139.7 132.08) (width 1) (layer F.Cu) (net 11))
 (segment (start 126.82 132.08) (end 123.96 134.94) (width 1) (layer F.Cu) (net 11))
 (segment (start 142.24 132.08) (end 126.82 132.08) (width 1) (layer F.Cu) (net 11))
 (segment (start 160.02 119.38) (end 160.02 132.08) (width 1) (layer B.Cu) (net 12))
 (segment (start 162.56 132.08) (end 160.02 132.08) (width 1) (layer B.Cu) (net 12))
 (segment (start 160.02 104.14) (end 157.48 106.68) (width 1) (layer B.Cu) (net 12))
 (segment (start 157.48 116.84) (end 160.02 119.38) (width 1) (layer B.Cu) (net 12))
 (segment (start 157.48 106.68) (end 157.48 116.84) (width 1) (layer B.Cu) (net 12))
 (segment (start 117.36 139.18) (end 117.36 139.34) (width 1) (layer F.Cu) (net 12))
 (segment (start 119.38 137.16) (end 117.36 139.18) (width 1) (layer F.Cu) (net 12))
 (segment (start 129.54 134.62) (end 127 137.16) (width 1) (layer F.Cu) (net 12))
 (segment (start 162.56 132.08) (end 149.540002 132.08) (width 1) (layer F.Cu) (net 12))
 (segment (start 137.16 137.16) (end 134.62 134.62) (width 1) (layer F.Cu) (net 12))
 (segment (start 144.460002 137.16) (end 137.16 137.16) (width 1) (layer F.Cu) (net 12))
 (segment (start 127 137.16) (end 119.38 137.16) (width 1) (layer F.Cu) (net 12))
 (segment (start 149.540002 132.08) (end 144.460002 137.16) (width 1) (layer F.Cu) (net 12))
 (segment (start 134.62 134.62) (end 129.54 134.62) (width 1) (layer F.Cu) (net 12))
 (segment (start 115.86 139.34) (end 114.66 138.14) (width 1) (layer F.Cu) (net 12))
 (segment (start 117.36 139.34) (end 115.86 139.34) (width 1) (layer F.Cu) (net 12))
 (segment (start 144.78 116.84) (end 144.78 121.92) (width 1) (layer B.Cu) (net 13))
 (segment (start 144.78 121.92) (end 142.24 121.92) (width 1) (layer B.Cu) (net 13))
 (segment (start 139.7 114.3) (end 142.24 116.84) (width 1) (layer B.Cu) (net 14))
 (segment (start 139.7 109.22) (end 139.7 114.3) (width 1) (layer B.Cu) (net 14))
 (segment (start 142.24 116.84) (end 149.86 109.22) (width 1) (layer B.Cu) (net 14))
 (segment (start 147.32 106.68) (end 147.32 109.22) (width 1) (layer B.Cu) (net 15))
 (segment (start 147.32 106.68) (end 149.86 104.14) (width 1) (layer B.Cu) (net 15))
 (segment (start 147.32 109.22) (end 144.78 109.22) (width 1) (layer B.Cu) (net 15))
 (segment (start 165.1 116.84) (end 165.1 121.92) (width 1) (layer B.Cu) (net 16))
 (segment (start 165.1 121.92) (end 162.56 121.92) (width 1) (layer B.Cu) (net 16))
 (segment (start 160.02 114.3) (end 160.02 109.22) (width 1) (layer B.Cu) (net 17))
 (segment (start 160.02 114.3) (end 162.56 116.84) (width 1) (layer B.Cu) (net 17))
 (segment (start 162.56 116.84) (end 170.18 109.22) (width 1) (layer B.Cu) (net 17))
 (segment (start 167.64 106.68) (end 167.64 109.22) (width 1) (layer B.Cu) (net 18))
 (segment (start 167.64 109.22) (end 165.1 109.22) (width 1) (layer B.Cu) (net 18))
 (segment (start 167.64 106.68) (end 170.18 104.14) (width 1) (layer B.Cu) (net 18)))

